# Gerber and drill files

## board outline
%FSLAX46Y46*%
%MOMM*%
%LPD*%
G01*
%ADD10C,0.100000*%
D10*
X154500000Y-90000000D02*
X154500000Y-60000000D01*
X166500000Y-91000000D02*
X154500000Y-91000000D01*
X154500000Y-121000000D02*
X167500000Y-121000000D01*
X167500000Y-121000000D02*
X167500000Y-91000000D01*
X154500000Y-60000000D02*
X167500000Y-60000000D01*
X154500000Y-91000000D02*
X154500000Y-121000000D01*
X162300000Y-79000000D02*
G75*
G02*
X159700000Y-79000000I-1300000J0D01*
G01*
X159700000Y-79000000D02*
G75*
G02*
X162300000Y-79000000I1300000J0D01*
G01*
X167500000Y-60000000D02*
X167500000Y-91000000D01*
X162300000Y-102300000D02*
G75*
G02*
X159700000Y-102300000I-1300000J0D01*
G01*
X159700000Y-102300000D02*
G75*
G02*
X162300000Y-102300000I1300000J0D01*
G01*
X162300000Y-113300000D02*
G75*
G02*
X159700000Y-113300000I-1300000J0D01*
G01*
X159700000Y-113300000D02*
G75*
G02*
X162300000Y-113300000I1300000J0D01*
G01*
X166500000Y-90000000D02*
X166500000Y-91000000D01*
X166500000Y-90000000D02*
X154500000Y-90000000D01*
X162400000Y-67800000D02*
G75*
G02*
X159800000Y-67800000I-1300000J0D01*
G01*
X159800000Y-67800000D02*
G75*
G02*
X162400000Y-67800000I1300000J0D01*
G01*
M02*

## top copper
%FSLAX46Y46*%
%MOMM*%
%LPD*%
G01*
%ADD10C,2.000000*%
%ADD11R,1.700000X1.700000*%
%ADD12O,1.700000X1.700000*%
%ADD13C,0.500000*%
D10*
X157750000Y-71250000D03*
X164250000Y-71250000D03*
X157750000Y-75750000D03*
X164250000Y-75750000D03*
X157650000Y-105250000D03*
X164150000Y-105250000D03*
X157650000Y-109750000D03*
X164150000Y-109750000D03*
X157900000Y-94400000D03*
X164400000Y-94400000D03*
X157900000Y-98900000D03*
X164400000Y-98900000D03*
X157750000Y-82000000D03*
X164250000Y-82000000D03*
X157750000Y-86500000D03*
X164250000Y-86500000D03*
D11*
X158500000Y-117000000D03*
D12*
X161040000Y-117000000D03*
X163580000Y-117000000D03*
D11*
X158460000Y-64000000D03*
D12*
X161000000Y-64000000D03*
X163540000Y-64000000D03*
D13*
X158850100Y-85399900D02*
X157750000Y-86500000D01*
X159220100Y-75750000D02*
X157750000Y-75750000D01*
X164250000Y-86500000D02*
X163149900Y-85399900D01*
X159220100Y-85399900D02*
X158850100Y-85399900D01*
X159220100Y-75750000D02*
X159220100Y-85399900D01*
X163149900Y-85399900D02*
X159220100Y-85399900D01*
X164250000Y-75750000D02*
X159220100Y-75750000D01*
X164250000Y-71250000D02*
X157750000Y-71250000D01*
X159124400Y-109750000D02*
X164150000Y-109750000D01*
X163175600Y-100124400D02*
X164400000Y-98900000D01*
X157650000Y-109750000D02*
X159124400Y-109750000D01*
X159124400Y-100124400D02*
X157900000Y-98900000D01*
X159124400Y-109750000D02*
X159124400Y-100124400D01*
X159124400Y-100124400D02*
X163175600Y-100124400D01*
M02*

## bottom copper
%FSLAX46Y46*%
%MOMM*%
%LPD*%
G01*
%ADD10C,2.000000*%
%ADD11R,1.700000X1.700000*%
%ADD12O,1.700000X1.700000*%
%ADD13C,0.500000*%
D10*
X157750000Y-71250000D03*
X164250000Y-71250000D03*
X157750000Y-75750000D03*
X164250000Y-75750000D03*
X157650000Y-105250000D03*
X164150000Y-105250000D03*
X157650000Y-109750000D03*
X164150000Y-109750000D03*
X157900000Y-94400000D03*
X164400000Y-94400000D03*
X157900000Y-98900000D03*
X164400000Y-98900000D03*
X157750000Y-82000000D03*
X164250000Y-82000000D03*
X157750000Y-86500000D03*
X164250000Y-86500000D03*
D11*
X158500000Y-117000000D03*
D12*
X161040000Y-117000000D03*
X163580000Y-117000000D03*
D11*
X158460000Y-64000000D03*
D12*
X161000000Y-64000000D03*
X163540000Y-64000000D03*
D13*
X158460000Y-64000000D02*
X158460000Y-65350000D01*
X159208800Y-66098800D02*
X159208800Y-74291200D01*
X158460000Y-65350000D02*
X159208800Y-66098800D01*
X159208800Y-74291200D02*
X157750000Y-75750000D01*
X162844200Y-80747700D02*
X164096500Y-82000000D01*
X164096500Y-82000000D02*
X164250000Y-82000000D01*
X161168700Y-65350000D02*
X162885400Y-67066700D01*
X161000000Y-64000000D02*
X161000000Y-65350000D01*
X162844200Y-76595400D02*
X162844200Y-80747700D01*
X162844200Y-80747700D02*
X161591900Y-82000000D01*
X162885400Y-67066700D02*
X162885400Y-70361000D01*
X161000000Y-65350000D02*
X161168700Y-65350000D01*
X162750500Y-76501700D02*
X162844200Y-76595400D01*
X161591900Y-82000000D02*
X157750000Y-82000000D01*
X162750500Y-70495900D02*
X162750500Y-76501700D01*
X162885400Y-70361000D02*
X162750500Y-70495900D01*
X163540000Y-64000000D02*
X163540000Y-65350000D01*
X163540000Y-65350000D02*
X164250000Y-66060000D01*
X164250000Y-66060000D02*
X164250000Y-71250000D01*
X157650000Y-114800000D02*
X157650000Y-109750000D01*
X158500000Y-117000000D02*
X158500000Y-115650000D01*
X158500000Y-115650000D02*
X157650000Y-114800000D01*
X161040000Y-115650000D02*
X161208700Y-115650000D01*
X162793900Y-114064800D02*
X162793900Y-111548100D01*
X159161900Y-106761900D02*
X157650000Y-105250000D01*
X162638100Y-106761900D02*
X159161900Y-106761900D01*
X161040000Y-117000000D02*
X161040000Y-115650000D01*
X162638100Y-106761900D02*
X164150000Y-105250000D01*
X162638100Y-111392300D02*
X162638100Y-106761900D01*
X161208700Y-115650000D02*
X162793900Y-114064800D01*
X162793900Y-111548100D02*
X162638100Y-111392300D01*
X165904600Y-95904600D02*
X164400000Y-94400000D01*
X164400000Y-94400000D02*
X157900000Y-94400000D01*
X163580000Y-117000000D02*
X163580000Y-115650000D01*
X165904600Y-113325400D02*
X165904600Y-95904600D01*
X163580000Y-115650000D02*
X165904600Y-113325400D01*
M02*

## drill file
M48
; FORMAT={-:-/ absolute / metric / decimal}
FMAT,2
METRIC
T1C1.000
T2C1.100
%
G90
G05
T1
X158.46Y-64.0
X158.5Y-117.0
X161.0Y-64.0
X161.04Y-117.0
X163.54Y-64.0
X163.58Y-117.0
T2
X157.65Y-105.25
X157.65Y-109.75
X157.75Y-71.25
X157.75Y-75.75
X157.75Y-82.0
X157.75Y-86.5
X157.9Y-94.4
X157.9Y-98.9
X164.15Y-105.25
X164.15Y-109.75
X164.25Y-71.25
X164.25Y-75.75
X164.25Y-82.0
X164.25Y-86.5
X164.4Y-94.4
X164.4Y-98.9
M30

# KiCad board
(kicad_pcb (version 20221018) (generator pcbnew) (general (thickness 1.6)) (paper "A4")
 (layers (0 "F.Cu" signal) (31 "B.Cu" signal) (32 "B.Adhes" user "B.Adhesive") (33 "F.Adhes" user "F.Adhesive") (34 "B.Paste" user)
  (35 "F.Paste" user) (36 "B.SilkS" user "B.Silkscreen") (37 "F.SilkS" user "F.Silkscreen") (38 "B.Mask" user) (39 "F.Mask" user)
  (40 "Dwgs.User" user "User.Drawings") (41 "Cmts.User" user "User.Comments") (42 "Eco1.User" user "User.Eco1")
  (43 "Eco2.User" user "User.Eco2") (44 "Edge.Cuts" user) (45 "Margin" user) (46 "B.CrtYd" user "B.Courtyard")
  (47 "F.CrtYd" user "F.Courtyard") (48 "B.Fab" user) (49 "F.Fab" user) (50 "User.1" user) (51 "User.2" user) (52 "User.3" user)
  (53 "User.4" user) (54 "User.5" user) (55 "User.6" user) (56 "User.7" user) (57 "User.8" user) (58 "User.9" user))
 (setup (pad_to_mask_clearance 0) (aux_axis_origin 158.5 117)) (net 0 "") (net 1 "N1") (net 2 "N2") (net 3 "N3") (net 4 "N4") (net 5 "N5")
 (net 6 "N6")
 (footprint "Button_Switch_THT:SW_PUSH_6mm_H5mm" (layer "F.Cu") (at 157.75 71.25)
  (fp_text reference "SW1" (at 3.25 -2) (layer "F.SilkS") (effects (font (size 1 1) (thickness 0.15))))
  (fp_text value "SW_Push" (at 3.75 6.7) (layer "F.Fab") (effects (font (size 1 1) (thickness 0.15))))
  (pad "1" thru_hole circle (at 0 0 90) (size 2 2) (drill 1.1) (layers "*.Cu" "*.Mask") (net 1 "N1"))
  (pad "1" thru_hole circle (at 6.5 0 90) (size 2 2) (drill 1.1) (layers "*.Cu" "*.Mask") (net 1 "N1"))
  (pad "2" thru_hole circle (at 0 4.5 90) (size 2 2) (drill 1.1) (layers "*.Cu" "*.Mask") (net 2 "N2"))
  (pad "2" thru_hole circle (at 6.5 4.5 90) (size 2 2) (drill 1.1) (layers "*.Cu" "*.Mask") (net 2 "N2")))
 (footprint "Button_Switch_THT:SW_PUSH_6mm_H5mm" (layer "F.Cu") (at 157.65 105.25)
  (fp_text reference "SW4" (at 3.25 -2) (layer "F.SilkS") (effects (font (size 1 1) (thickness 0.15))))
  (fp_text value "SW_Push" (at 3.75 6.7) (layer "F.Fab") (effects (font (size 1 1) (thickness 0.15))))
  (pad "1" thru_hole circle (at 0 0 90) (size 2 2) (drill 1.1) (layers "*.Cu" "*.Mask") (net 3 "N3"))
  (pad "1" thru_hole circle (at 6.5 0 90) (size 2 2) (drill 1.1) (layers "*.Cu" "*.Mask") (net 3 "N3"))
  (pad "2" thru_hole circle (at 0 4.5 90) (size 2 2) (drill 1.1) (layers "*.Cu" "*.Mask") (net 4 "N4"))
  (pad "2" thru_hole circle (at 6.5 4.5 90) (size 2 2) (drill 1.1) (layers "*.Cu" "*.Mask") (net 4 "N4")))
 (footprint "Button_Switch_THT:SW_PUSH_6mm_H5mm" (layer "F.Cu") (at 157.9 94.4)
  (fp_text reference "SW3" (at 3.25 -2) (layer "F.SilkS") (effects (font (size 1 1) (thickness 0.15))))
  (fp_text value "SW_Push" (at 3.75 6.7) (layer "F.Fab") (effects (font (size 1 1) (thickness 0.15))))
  (pad "1" thru_hole circle (at 0 0 90) (size 2 2) (drill 1.1) (layers "*.Cu" "*.Mask") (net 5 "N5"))
  (pad "1" thru_hole circle (at 6.5 0 90) (size 2 2) (drill 1.1) (layers "*.Cu" "*.Mask") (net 5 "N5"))
  (pad "2" thru_hole circle (at 0 4.5 90) (size 2 2) (drill 1.1) (layers "*.Cu" "*.Mask") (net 4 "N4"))
  (pad "2" thru_hole circle (at 6.5 4.5 90) (size 2 2) (drill 1.1) (layers "*.Cu" "*.Mask") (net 4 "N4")))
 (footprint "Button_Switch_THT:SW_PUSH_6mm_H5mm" (layer "F.Cu") (at 157.75 82)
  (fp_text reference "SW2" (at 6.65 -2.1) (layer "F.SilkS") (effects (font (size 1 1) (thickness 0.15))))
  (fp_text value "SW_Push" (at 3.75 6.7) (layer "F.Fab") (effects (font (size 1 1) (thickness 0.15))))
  (pad "1" thru_hole circle (at 0 0 90) (size 2 2) (drill 1.1) (layers "*.Cu" "*.Mask") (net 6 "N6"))
  (pad "1" thru_hole circle (at 6.5 0 90) (size 2 2) (drill 1.1) (layers "*.Cu" "*.Mask") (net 6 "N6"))
  (pad "2" thru_hole circle (at 0 4.5 90) (size 2 2) (drill 1.1) (layers "*.Cu" "*.Mask") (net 2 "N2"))
  (pad "2" thru_hole circle (at 6.5 4.5 90) (size 2 2) (drill 1.1) (layers "*.Cu" "*.Mask") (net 2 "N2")))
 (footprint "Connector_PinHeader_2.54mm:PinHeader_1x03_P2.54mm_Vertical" (layer "F.Cu") (at 158.5 117 90)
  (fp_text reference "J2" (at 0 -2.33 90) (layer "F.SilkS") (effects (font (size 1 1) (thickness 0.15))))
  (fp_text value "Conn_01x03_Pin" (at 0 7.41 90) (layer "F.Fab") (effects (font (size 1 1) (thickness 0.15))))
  (pad "1" thru_hole rect (at 0 0 90) (size 1.7 1.7) (drill 1) (layers "*.Cu" "*.Mask") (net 4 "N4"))
  (pad "2" thru_hole oval (at 0 2.54 90) (size 1.7 1.7) (drill 1) (layers "*.Cu" "*.Mask") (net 3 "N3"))
  (pad "3" thru_hole oval (at 0 5.08 90) (size 1.7 1.7) (drill 1) (layers "*.Cu" "*.Mask") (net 5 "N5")))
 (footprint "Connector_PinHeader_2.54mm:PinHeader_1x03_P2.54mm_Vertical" (layer "F.Cu") (at 158.46 64 90)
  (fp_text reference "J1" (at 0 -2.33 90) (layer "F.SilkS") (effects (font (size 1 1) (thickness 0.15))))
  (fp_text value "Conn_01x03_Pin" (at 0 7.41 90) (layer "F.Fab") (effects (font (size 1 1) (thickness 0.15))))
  (pad "1" thru_hole rect (at 0 0 90) (size 1.7 1.7) (drill 1) (layers "*.Cu" "*.Mask") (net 2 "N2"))
  (pad "2" thru_hole oval (at 0 2.54 90) (size 1.7 1.7) (drill 1) (layers "*.Cu" "*.Mask") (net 6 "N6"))
  (pad "3" thru_hole oval (at 0 5.08 90) (size 1.7 1.7) (drill 1) (layers "*.Cu" "*.Mask") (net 1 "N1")))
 (gr_line (start 154.5 90) (end 154.5 60) (stroke (width 0.1) (type default)) (layer "Edge.Cuts"))
 (gr_line (start 166.5 91) (end 154.5 91) (stroke (width 0.1) (type default)) (layer "Edge.Cuts"))
 (gr_line (start 154.5 121) (end 167.5 121) (stroke (width 0.1) (type default)) (layer "Edge.Cuts"))
 (gr_line (start 167.5 121) (end 167.5 91) (stroke (width 0.1) (type default)) (layer "Edge.Cuts"))
 (gr_line (start 154.5 60) (end 167.5 60) (stroke (width 0.1) (type default)) (layer "Edge.Cuts"))
 (gr_line (start 154.5 91) (end 154.5 121) (stroke (width 0.1) (type default)) (layer "Edge.Cuts"))
 (gr_circle (center 161 79) (end 162.3 79) (stroke (width 0.1) (type default)) (fill none) (layer "Edge.Cuts"))
 (gr_line (start 167.5 60) (end 167.5 91) (stroke (width 0.1) (type default)) (layer "Edge.Cuts"))
 (gr_circle (center 161 102.3) (end 162.3 102.3) (stroke (width 0.1) (type default)) (fill none) (layer "Edge.Cuts"))
 (gr_circle (center 161 113.3) (end 162.3 113.3) (stroke (width 0.1) (type default)) (fill none) (layer "Edge.Cuts"))
 (gr_line (start 166.5 90) (end 166.5 91) (stroke (width 0.1) (type default)) (layer "Edge.Cuts"))
 (gr_line (start 166.5 90) (end 154.5 90) (stroke (width 0.1) (type default)) (layer "Edge.Cuts"))
 (gr_circle (center 161.1 67.8) (end 162.4 67.8) (stroke (width 0.1) (type default)) (fill none) (layer "Edge.Cuts"))
 (segment (start 158.8501 85.3999) (end 157.75 86.5) (width 0.5) (layer "F.Cu") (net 2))
 (segment (start 159.2201 75.75) (end 157.75 75.75) (width 0.5) (layer "F.Cu") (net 2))
 (segment (start 164.25 86.5) (end 163.1499 85.3999) (width 0.5) (layer "F.Cu") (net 2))
 (segment (start 159.2201 85.3999) (end 158.8501 85.3999) (width 0.5) (layer "F.Cu") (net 2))
 (segment (start 159.2201 75.75) (end 159.2201 85.3999) (width 0.5) (layer "F.Cu") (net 2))
 (segment (start 163.1499 85.3999) (end 159.2201 85.3999) (width 0.5) (layer "F.Cu") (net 2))
 (segment (start 164.25 75.75) (end 159.2201 75.75) (width 0.5) (layer "F.Cu") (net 2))
 (segment (start 158.46 64) (end 158.46 65.35) (width 0.5) (layer "B.Cu") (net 2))
 (segment (start 159.2088 66.0988) (end 159.2088 74.2912) (width 0.5) (layer "B.Cu") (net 2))
 (segment (start 158.46 65.35) (end 159.2088 66.0988) (width 0.5) (layer "B.Cu") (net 2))
 (segment (start 159.2088 74.2912) (end 157.75 75.75) (width 0.5) (layer "B.Cu") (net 2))
 (segment (start 162.8442 80.7477) (end 164.0965 82) (width 0.5) (layer "B.Cu") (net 6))
 (segment (start 164.0965 82) (end 164.25 82) (width 0.5) (layer "B.Cu") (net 6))
 (segment (start 161.1687 65.35) (end 162.8854 67.0667) (width 0.5) (layer "B.Cu") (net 6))
 (segment (start 161 64) (end 161 65.35) (width 0.5) (layer "B.Cu") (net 6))
 (segment (start 162.8442 76.5954) (end 162.8442 80.7477) (width 0.5) (layer "B.Cu") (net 6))
 (segment (start 162.8442 80.7477) (end 161.5919 82) (width 0.5) (layer "B.Cu") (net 6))
 (segment (start 162.8854 67.0667) (end 162.8854 70.361) (width 0.5) (layer "B.Cu") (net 6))
 (segment (start 161 65.35) (end 161.1687 65.35) (width 0.5) (layer "B.Cu") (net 6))
 (segment (start 162.7505 76.5017) (end 162.8442 76.5954) (width 0.5) (layer "B.Cu") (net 6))
 (segment (start 161.5919 82) (end 157.75 82) (width 0.5) (layer "B.Cu") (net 6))
 (segment (start 162.7505 70.4959) (end 162.7505 76.5017) (width 0.5) (layer "B.Cu") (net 6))
 (segment (start 162.8854 70.361) (end 162.7505 70.4959) (width 0.5) (layer "B.Cu") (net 6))
 (segment (start 164.25 71.25) (end 157.75 71.25) (width 0.5) (layer "F.Cu") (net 1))
 (segment (start 163.54 64) (end 163.54 65.35) (width 0.5) (layer "B.Cu") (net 1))
 (segment (start 163.54 65.35) (end 164.25 66.06) (width 0.5) (layer "B.Cu") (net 1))
 (segment (start 164.25 66.06) (end 164.25 71.25) (width 0.5) (layer "B.Cu") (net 1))
 (segment (start 159.1244 109.75) (end 164.15 109.75) (width 0.5) (layer "F.Cu") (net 4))
 (segment (start 163.1756 100.1244) (end 164.4 98.9) (width 0.5) (layer "F.Cu") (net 4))
 (segment (start 157.65 109.75) (end 159.1244 109.75) (width 0.5) (layer "F.Cu") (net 4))
 (segment (start 159.1244 100.1244) (end 157.9 98.9) (width 0.5) (layer "F.Cu") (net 4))
 (segment (start 159.1244 109.75) (end 159.1244 100.1244) (width 0.5) (layer "F.Cu") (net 4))
 (segment (start 159.1244 100.1244) (end 163.1756 100.1244) (width 0.5) (layer "F.Cu") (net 4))
 (segment (start 157.65 114.8) (end 157.65 109.75) (width 0.5) (layer "B.Cu") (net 4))
 (segment (start 158.5 117) (end 158.5 115.65) (width 0.5) (layer "B.Cu") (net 4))
 (segment (start 158.5 115.65) (end 157.65 114.8) (width 0.5) (layer "B.Cu") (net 4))
 (segment (start 161.04 115.65) (end 161.2087 115.65) (width 0.5) (layer "B.Cu") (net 3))
 (segment (start 162.7939 114.0648) (end 162.7939 111.5481) (width 0.5) (layer "B.Cu") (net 3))
 (segment (start 159.1619 106.7619) (end 157.65 105.25) (width 0.5) (layer "B.Cu") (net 3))
 (segment (start 162.6381 106.7619) (end 159.1619 106.7619) (width 0.5) (layer "B.Cu") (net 3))
 (segment (start 161.04 117) (end 161.04 115.65) (width 0.5) (layer "B.Cu") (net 3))
 (segment (start 162.6381 106.7619) (end 164.15 105.25) (width 0.5) (layer "B.Cu") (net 3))
 (segment (start 162.6381 111.3923) (end 162.6381 106.7619) (width 0.5) (layer "B.Cu") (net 3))
 (segment (start 161.2087 115.65) (end 162.7939 114.0648) (width 0.5) (layer "B.Cu") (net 3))
 (segment (start 162.7939 111.5481) (end 162.6381 111.3923) (width 0.5) (layer "B.Cu") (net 3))
 (segment (start 165.9046 95.9046) (end 164.4 94.4) (width 0.5) (layer "B.Cu") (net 5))
 (segment (start 164.4 94.4) (end 157.9 94.4) (width 0.5) (layer "B.Cu") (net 5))
 (segment (start 163.58 117) (end 163.58 115.65) (width 0.5) (layer "B.Cu") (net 5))
 (segment (start 165.9046 113.3254) (end 165.9046 95.9046) (width 0.5) (layer "B.Cu") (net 5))
 (segment (start 163.58 115.65) (end 165.9046 113.3254) (width 0.5) (layer "B.Cu") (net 5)))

